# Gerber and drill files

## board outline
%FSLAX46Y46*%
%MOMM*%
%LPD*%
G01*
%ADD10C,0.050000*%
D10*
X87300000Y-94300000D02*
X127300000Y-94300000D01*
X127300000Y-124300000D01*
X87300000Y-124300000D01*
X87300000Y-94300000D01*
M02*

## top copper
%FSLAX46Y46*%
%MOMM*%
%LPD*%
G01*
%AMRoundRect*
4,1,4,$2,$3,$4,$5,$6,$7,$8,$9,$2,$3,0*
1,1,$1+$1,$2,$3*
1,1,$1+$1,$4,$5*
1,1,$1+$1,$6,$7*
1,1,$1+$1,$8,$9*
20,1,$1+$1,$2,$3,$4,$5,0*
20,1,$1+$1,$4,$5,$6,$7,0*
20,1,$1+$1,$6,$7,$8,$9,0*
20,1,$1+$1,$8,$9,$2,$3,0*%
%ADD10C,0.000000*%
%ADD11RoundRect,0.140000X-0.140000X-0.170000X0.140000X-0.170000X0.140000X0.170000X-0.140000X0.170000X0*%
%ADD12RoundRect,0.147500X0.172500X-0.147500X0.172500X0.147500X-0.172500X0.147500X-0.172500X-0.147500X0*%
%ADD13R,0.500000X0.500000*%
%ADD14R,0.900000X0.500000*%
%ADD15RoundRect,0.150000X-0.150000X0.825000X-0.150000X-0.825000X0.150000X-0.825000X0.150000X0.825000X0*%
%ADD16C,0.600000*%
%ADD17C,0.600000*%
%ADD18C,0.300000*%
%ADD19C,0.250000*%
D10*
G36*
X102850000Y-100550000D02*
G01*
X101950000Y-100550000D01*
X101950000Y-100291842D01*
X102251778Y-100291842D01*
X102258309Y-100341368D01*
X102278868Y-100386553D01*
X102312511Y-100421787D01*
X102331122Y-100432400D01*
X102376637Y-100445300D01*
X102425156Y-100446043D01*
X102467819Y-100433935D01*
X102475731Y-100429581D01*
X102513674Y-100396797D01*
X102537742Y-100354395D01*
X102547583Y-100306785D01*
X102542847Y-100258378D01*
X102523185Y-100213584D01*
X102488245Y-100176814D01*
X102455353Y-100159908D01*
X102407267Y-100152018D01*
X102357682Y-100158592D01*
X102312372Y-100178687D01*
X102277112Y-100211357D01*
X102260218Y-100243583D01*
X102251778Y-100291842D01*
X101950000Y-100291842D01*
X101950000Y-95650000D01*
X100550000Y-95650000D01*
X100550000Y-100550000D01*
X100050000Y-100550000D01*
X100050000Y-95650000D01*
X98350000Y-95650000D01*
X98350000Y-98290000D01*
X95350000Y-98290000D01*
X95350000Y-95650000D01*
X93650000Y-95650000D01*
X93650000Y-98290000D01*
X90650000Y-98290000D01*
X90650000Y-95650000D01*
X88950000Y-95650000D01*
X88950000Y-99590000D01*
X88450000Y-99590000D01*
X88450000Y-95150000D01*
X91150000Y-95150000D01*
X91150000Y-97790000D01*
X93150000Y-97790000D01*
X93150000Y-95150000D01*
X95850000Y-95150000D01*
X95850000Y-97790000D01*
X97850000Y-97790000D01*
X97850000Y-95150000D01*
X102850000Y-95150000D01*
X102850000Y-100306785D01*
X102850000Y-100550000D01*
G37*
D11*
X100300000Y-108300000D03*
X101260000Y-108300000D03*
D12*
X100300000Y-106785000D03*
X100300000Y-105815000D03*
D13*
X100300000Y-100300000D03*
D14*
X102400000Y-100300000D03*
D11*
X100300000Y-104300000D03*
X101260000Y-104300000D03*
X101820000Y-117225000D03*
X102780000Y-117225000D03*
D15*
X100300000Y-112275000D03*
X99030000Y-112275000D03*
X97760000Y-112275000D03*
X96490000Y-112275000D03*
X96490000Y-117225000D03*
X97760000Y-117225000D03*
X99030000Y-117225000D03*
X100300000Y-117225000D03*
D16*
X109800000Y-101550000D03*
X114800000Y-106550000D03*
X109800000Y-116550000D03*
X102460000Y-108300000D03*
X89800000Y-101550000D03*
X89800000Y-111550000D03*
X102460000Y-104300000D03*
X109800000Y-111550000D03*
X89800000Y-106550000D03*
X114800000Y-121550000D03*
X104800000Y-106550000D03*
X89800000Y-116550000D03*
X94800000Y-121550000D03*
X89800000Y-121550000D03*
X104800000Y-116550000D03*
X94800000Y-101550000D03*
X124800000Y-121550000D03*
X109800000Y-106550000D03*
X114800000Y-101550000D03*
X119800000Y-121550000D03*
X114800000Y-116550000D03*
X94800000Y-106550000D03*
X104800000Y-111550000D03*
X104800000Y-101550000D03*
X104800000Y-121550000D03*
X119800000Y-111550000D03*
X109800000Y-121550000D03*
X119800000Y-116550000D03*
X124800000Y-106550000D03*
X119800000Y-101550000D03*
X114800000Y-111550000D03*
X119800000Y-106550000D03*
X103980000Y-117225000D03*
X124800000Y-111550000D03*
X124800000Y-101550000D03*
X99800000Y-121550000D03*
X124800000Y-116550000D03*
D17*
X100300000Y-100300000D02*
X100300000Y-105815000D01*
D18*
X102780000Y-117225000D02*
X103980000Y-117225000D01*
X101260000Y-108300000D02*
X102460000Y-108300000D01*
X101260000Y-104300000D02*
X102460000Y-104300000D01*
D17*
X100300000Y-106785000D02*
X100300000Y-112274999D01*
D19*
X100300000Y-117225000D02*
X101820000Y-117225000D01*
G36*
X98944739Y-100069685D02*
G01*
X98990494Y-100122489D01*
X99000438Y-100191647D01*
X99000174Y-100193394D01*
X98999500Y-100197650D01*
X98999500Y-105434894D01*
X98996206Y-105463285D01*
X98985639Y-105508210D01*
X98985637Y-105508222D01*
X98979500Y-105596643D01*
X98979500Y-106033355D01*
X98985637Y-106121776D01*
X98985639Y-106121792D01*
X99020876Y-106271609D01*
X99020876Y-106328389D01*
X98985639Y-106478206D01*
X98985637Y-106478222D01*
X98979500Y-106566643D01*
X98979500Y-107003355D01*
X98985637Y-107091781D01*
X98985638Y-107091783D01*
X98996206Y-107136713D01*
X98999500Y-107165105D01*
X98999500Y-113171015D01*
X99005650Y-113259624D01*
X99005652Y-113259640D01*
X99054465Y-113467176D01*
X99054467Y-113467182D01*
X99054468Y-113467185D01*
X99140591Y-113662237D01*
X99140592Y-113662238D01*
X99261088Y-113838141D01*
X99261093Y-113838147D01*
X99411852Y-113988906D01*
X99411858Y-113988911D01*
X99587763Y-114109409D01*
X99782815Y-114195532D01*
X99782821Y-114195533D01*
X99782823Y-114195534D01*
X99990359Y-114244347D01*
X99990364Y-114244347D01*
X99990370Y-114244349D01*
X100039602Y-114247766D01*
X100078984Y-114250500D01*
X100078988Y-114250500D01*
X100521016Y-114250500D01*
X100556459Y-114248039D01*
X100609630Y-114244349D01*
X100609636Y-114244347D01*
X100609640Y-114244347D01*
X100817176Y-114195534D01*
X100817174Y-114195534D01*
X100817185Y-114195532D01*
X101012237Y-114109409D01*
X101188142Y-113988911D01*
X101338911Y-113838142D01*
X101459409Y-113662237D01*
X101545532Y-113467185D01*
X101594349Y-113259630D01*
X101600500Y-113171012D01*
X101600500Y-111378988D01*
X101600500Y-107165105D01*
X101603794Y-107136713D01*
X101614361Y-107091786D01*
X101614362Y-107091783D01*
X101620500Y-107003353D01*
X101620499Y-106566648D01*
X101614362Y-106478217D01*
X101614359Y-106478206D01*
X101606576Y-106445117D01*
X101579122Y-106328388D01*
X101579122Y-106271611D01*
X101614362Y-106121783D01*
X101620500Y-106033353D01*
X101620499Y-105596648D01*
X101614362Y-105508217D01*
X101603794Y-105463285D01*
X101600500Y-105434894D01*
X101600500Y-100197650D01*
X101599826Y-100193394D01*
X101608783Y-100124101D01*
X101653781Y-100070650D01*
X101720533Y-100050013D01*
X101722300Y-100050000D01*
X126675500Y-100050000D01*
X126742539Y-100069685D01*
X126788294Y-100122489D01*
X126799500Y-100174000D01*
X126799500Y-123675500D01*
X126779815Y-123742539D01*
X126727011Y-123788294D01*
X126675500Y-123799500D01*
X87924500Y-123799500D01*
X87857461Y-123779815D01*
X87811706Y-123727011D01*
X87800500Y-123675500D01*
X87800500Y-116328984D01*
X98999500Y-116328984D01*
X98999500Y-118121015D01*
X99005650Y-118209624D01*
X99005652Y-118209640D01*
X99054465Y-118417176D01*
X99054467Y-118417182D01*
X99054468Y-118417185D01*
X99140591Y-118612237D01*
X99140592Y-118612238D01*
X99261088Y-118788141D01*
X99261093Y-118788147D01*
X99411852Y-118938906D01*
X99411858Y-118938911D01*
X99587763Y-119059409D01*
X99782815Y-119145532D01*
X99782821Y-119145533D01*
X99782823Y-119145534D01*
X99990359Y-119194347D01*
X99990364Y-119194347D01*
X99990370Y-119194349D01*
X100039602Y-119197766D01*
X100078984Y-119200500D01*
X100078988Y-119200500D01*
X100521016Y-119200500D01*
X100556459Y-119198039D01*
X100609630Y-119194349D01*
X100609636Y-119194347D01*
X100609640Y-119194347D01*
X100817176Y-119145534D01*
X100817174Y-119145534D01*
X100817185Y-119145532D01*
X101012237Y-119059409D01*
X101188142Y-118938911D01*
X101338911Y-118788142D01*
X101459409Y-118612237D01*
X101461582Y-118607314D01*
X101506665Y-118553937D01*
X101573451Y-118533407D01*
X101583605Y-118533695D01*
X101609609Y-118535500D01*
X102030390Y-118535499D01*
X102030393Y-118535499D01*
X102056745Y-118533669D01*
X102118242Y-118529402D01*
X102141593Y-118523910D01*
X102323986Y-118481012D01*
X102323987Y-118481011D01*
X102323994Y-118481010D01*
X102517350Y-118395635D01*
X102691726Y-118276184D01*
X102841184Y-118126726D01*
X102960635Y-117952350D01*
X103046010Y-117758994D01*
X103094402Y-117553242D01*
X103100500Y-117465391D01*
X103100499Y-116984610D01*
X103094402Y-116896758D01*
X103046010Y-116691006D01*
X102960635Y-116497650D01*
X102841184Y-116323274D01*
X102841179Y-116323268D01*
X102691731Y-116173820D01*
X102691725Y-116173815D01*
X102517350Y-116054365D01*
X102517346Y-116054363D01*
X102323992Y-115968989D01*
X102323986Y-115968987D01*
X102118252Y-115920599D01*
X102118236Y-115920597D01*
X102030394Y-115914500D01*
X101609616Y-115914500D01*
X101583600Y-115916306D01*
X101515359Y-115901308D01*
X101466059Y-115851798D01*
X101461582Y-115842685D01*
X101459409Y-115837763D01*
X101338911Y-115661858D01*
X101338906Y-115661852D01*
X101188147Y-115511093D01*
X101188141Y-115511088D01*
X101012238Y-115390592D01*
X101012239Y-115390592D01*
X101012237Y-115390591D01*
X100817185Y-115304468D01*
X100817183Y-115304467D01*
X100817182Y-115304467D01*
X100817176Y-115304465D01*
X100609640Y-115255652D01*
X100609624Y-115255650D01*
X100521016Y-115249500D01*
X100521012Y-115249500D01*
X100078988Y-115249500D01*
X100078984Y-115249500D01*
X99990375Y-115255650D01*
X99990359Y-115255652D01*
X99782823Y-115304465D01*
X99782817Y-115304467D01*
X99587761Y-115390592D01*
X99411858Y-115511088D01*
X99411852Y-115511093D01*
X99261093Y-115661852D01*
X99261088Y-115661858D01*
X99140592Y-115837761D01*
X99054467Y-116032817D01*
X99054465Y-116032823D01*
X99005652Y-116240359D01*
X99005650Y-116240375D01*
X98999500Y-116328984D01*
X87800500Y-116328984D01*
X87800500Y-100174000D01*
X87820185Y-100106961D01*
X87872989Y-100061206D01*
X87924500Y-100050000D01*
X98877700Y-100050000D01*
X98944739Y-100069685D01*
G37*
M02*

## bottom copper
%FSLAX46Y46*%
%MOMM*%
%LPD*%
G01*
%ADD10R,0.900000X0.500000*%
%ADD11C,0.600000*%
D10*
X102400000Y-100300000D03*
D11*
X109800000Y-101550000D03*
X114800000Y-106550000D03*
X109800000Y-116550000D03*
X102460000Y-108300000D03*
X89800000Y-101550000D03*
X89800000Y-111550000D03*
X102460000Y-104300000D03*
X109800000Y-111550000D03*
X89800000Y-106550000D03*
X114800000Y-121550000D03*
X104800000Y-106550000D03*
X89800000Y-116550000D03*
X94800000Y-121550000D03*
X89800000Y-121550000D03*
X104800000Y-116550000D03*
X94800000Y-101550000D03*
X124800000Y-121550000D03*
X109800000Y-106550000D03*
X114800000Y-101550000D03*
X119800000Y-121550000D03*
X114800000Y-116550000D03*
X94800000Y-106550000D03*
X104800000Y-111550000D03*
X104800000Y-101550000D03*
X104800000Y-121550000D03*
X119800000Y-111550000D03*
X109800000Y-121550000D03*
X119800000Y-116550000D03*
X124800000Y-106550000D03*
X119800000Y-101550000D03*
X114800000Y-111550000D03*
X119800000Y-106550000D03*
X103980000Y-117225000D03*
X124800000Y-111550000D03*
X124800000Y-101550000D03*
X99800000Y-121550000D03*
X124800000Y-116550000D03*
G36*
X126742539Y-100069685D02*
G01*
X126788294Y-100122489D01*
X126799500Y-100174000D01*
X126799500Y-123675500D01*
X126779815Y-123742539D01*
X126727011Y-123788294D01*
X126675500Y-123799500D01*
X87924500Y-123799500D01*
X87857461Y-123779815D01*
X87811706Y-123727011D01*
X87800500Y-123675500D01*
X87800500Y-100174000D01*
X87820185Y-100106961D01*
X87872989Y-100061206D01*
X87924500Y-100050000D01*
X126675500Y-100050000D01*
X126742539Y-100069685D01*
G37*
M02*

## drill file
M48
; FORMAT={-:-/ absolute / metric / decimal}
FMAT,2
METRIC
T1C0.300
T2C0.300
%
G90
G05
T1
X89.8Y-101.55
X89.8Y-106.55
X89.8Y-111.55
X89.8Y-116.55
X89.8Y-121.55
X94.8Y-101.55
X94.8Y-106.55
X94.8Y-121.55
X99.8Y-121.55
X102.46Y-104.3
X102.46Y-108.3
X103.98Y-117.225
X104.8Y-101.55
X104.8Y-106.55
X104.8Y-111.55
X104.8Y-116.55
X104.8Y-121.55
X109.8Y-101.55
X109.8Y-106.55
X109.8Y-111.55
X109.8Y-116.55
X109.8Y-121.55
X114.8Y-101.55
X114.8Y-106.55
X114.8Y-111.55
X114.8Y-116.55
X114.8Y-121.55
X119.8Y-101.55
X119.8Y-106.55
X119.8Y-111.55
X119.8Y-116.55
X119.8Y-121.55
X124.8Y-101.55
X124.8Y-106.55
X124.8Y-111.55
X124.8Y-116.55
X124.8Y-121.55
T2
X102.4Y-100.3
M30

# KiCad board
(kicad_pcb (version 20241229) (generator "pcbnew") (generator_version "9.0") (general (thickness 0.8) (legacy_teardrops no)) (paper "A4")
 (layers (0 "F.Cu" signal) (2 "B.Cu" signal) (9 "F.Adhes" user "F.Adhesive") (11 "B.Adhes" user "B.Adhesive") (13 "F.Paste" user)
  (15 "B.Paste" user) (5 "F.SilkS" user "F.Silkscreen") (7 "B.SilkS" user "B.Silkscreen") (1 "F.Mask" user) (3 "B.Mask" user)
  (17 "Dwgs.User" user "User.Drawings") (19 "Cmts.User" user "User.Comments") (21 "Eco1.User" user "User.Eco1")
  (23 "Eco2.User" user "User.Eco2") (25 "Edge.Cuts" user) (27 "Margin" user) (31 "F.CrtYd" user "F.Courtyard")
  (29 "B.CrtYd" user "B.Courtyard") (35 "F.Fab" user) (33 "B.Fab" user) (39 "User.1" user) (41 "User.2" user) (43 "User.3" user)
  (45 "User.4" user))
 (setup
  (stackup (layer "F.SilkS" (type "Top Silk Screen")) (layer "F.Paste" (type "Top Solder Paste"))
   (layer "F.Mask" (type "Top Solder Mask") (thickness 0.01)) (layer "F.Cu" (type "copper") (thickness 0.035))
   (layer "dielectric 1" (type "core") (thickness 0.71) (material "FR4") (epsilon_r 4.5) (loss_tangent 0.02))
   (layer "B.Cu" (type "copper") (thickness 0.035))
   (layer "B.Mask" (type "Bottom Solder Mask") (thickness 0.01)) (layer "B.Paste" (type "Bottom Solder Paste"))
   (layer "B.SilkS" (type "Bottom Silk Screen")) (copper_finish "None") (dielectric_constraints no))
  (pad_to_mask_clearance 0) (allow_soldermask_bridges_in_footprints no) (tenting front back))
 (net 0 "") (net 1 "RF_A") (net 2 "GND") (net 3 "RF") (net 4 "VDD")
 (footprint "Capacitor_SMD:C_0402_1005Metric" (layer "F.Cu") (at 100.78 108.3)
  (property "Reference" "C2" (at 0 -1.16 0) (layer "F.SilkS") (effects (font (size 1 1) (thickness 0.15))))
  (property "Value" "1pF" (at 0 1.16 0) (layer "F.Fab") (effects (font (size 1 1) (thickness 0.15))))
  (pad "1" smd roundrect (at -0.48 0) (size 0.56 0.62) (layers "F.Cu" "F.Mask" "F.Paste") (roundrect_rratio 0.25) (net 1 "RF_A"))
  (pad "2" smd roundrect (at 0.48 0) (size 0.56 0.62) (layers "F.Cu" "F.Mask" "F.Paste") (roundrect_rratio 0.25) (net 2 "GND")))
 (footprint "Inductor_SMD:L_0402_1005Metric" (layer "F.Cu") (at 100.3 106.3 90)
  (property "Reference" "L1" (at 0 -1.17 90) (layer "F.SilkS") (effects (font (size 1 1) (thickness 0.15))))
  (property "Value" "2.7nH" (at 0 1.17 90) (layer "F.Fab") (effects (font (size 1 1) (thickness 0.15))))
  (pad "1" smd roundrect (at -0.485 0 90) (size 0.59 0.64) (layers "F.Cu" "F.Mask" "F.Paste") (roundrect_rratio 0.25) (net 1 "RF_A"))
  (pad "2" smd roundrect (at 0.485 0 90) (size 0.59 0.64) (layers "F.Cu" "F.Mask" "F.Paste") (roundrect_rratio 0.25) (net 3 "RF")))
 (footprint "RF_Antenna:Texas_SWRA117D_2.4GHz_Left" (layer "F.Cu") (at 100.3 100.3)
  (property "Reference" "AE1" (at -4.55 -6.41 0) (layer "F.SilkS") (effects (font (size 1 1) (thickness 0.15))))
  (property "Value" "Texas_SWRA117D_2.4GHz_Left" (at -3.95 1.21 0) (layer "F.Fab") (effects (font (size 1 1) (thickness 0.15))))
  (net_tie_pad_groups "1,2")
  (fp_poly
   (pts (xy -2.45 -2.51) (xy -4.45 -2.51) (xy -4.45 -5.15) (xy -7.15 -5.15) (xy -7.15 -2.51) (xy -9.15 -2.51) (xy -9.15 -5.15)
    (xy -11.85 -5.15) (xy -11.85 -0.71) (xy -11.35 -0.71) (xy -11.35 -4.65) (xy -9.65 -4.65) (xy -9.65 -2.01) (xy -6.65 -2.01)
    (xy -6.65 -4.65) (xy -4.95 -4.65) (xy -4.95 -2.01) (xy -1.95 -2.01) (xy -1.95 -4.65) (xy -0.25 -4.65) (xy -0.25 0.25) (xy 0.25 0.25)
    (xy 0.25 -4.65) (xy 1.65 -4.65) (xy 1.65 0.25) (xy 2.55 0.25) (xy 2.55 0.006785) (xy 2.247583 0.006785) (xy 2.237742 0.054395)
    (xy 2.213674 0.096797) (xy 2.175731 0.129581) (xy 2.167819 0.133935) (xy 2.125156 0.146043) (xy 2.076637 0.1453) (xy 2.031122 0.1324)
    (xy 2.012511 0.121787) (xy 1.978868 0.086553) (xy 1.958309 0.041368) (xy 1.951778 -0.008158) (xy 1.960218 -0.056417)
    (xy 1.977112 -0.088643) (xy 2.012372 -0.121313) (xy 2.057682 -0.141408) (xy 2.107267 -0.147982) (xy 2.155353 -0.140092)
    (xy 2.188245 -0.123186) (xy 2.223185 -0.086416) (xy 2.242847 -0.041622) (xy 2.247583 0.006785) (xy 2.55 0.006785) (xy 2.55 -5.15)
    (xy -2.45 -5.15) (xy -2.45 -2.51))
   (stroke (width 0) (type solid)) (fill yes) (layer "F.Cu"))
  (pad "1" connect rect (at 0 0) (size 0.5 0.5) (layers "F.Cu") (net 3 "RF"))
  (pad "2" thru_hole rect (at 2.1 0) (size 0.9 0.5) (drill 0.3) (layers "*.Cu") (remove_unused_layers no) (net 2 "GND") (zone_connect 2)))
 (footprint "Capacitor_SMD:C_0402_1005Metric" (layer "F.Cu") (at 100.78 104.3)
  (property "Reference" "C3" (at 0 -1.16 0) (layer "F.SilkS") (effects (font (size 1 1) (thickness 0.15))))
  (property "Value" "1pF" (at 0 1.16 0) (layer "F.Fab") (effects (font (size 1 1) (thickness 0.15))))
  (pad "1" smd roundrect (at -0.48 0) (size 0.56 0.62) (layers "F.Cu" "F.Mask" "F.Paste") (roundrect_rratio 0.25) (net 3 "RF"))
  (pad "2" smd roundrect (at 0.48 0) (size 0.56 0.62) (layers "F.Cu" "F.Mask" "F.Paste") (roundrect_rratio 0.25) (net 2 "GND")))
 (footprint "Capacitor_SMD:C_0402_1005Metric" (layer "F.Cu") (at 102.3 117.225)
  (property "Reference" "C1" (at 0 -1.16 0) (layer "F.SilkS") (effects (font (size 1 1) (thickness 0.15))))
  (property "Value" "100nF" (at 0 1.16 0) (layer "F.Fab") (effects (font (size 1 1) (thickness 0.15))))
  (pad "1" smd roundrect (at -0.48 0) (size 0.56 0.62) (layers "F.Cu" "F.Mask" "F.Paste") (roundrect_rratio 0.25) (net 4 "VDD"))
  (pad "2" smd roundrect (at 0.48 0) (size 0.56 0.62) (layers "F.Cu" "F.Mask" "F.Paste") (roundrect_rratio 0.25) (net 2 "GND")))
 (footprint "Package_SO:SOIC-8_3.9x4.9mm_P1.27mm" (layer "F.Cu") (at 98.395 114.75 -90)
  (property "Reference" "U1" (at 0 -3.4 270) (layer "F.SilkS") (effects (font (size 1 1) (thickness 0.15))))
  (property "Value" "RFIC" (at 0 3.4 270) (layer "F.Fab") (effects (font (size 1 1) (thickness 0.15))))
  (pad "1" smd roundrect (at -2.475 -1.905 270) (size 1.95 0.6) (layers "F.Cu" "F.Mask" "F.Paste") (roundrect_rratio 0.25) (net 1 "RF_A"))
  (pad "2" smd roundrect (at -2.475 -0.635 270) (size 1.95 0.6) (layers "F.Cu" "F.Mask" "F.Paste") (roundrect_rratio 0.25) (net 2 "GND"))
  (pad "3" smd roundrect (at -2.475 0.635 270) (size 1.95 0.6) (layers "F.Cu" "F.Mask" "F.Paste") (roundrect_rratio 0.25) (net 2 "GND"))
  (pad "4" smd roundrect (at -2.475 1.905 270) (size 1.95 0.6) (layers "F.Cu" "F.Mask" "F.Paste") (roundrect_rratio 0.25) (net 2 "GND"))
  (pad "5" smd roundrect (at 2.475 1.905 270) (size 1.95 0.6) (layers "F.Cu" "F.Mask" "F.Paste") (roundrect_rratio 0.25) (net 2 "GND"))
  (pad "6" smd roundrect (at 2.475 0.635 270) (size 1.95 0.6) (layers "F.Cu" "F.Mask" "F.Paste") (roundrect_rratio 0.25) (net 2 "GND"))
  (pad "7" smd roundrect (at 2.475 -0.635 270) (size 1.95 0.6) (layers "F.Cu" "F.Mask" "F.Paste") (roundrect_rratio 0.25) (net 2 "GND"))
  (pad "8" smd roundrect (at 2.475 -1.905 270) (size 1.95 0.6) (layers "F.Cu" "F.Mask" "F.Paste") (roundrect_rratio 0.25) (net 4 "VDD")))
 (gr_rect (start 87.3 94.3) (end 127.3 124.3) (stroke (width 0.05) (type default)) (fill no) (layer "Edge.Cuts"))
 (segment (start 100.3 100.3) (end 100.3 105.815) (width 0.6) (layer "F.Cu") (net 3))
 (segment (start 102.78 117.225) (end 103.98 117.225) (width 0.3) (layer "F.Cu") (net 2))
 (segment (start 101.26 108.3) (end 102.46 108.3) (width 0.3) (layer "F.Cu") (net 2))
 (segment (start 101.26 104.3) (end 102.46 104.3) (width 0.3) (layer "F.Cu") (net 2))
 (via (at 109.8 101.55) (size 0.6) (drill 0.3) (layers "F.Cu" "B.Cu") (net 2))
 (via (at 114.8 106.55) (size 0.6) (drill 0.3) (layers "F.Cu" "B.Cu") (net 2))
 (via (at 109.8 116.55) (size 0.6) (drill 0.3) (layers "F.Cu" "B.Cu") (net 2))
 (via (at 102.46 108.3) (size 0.6) (drill 0.3) (layers "F.Cu" "B.Cu") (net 2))
 (via (at 89.8 101.55) (size 0.6) (drill 0.3) (layers "F.Cu" "B.Cu") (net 2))
 (via (at 89.8 111.55) (size 0.6) (drill 0.3) (layers "F.Cu" "B.Cu") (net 2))
 (via (at 102.46 104.3) (size 0.6) (drill 0.3) (layers "F.Cu" "B.Cu") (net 2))
 (via (at 109.8 111.55) (size 0.6) (drill 0.3) (layers "F.Cu" "B.Cu") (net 2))
 (via (at 89.8 106.55) (size 0.6) (drill 0.3) (layers "F.Cu" "B.Cu") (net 2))
 (via (at 114.8 121.55) (size 0.6) (drill 0.3) (layers "F.Cu" "B.Cu") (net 2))
 (via (at 104.8 106.55) (size 0.6) (drill 0.3) (layers "F.Cu" "B.Cu") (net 2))
 (via (at 89.8 116.55) (size 0.6) (drill 0.3) (layers "F.Cu" "B.Cu") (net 2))
 (via (at 94.8 121.55) (size 0.6) (drill 0.3) (layers "F.Cu" "B.Cu") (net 2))
 (via (at 89.8 121.55) (size 0.6) (drill 0.3) (layers "F.Cu" "B.Cu") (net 2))
 (via (at 104.8 116.55) (size 0.6) (drill 0.3) (layers "F.Cu" "B.Cu") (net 2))
 (via (at 94.8 101.55) (size 0.6) (drill 0.3) (layers "F.Cu" "B.Cu") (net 2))
 (via (at 124.8 121.55) (size 0.6) (drill 0.3) (layers "F.Cu" "B.Cu") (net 2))
 (via (at 109.8 106.55) (size 0.6) (drill 0.3) (layers "F.Cu" "B.Cu") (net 2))
 (via (at 114.8 101.55) (size 0.6) (drill 0.3) (layers "F.Cu" "B.Cu") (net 2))
 (via (at 119.8 121.55) (size 0.6) (drill 0.3) (layers "F.Cu" "B.Cu") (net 2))
 (via (at 114.8 116.55) (size 0.6) (drill 0.3) (layers "F.Cu" "B.Cu") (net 2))
 (via (at 94.8 106.55) (size 0.6) (drill 0.3) (layers "F.Cu" "B.Cu") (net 2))
 (via (at 104.8 111.55) (size 0.6) (drill 0.3) (layers "F.Cu" "B.Cu") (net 2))
 (via (at 104.8 101.55) (size 0.6) (drill 0.3) (layers "F.Cu" "B.Cu") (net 2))
 (via (at 104.8 121.55) (size 0.6) (drill 0.3) (layers "F.Cu" "B.Cu") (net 2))
 (via (at 119.8 111.55) (size 0.6) (drill 0.3) (layers "F.Cu" "B.Cu") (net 2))
 (via (at 109.8 121.55) (size 0.6) (drill 0.3) (layers "F.Cu" "B.Cu") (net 2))
 (via (at 119.8 116.55) (size 0.6) (drill 0.3) (layers "F.Cu" "B.Cu") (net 2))
 (via (at 124.8 106.55) (size 0.6) (drill 0.3) (layers "F.Cu" "B.Cu") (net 2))
 (via (at 119.8 101.55) (size 0.6) (drill 0.3) (layers "F.Cu" "B.Cu") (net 2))
 (via (at 114.8 111.55) (size 0.6) (drill 0.3) (layers "F.Cu" "B.Cu") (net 2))
 (via (at 119.8 106.55) (size 0.6) (drill 0.3) (layers "F.Cu" "B.Cu") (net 2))
 (via (at 103.98 117.225) (size 0.6) (drill 0.3) (layers "F.Cu" "B.Cu") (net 2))
 (via (at 124.8 111.55) (size 0.6) (drill 0.3) (layers "F.Cu" "B.Cu") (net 2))
 (via (at 124.8 101.55) (size 0.6) (drill 0.3) (layers "F.Cu" "B.Cu") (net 2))
 (via (at 99.8 121.55) (size 0.6) (drill 0.3) (layers "F.Cu" "B.Cu") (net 2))
 (via (at 124.8 116.55) (size 0.6) (drill 0.3) (layers "F.Cu" "B.Cu") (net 2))
 (segment (start 100.3 106.785) (end 100.3 112.274999) (width 0.6) (layer "F.Cu") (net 1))
 (segment (start 100.3 117.225) (end 101.82 117.225) (width 0.25) (layer "F.Cu") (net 4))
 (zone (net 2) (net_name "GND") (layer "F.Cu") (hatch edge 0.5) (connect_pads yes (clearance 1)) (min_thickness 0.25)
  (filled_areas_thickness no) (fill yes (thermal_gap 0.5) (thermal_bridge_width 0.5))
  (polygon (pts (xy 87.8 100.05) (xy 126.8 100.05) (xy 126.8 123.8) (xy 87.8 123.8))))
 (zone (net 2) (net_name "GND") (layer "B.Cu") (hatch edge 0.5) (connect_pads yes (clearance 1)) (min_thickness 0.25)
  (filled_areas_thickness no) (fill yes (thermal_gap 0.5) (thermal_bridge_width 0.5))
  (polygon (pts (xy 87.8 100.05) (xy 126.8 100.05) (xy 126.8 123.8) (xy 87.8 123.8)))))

